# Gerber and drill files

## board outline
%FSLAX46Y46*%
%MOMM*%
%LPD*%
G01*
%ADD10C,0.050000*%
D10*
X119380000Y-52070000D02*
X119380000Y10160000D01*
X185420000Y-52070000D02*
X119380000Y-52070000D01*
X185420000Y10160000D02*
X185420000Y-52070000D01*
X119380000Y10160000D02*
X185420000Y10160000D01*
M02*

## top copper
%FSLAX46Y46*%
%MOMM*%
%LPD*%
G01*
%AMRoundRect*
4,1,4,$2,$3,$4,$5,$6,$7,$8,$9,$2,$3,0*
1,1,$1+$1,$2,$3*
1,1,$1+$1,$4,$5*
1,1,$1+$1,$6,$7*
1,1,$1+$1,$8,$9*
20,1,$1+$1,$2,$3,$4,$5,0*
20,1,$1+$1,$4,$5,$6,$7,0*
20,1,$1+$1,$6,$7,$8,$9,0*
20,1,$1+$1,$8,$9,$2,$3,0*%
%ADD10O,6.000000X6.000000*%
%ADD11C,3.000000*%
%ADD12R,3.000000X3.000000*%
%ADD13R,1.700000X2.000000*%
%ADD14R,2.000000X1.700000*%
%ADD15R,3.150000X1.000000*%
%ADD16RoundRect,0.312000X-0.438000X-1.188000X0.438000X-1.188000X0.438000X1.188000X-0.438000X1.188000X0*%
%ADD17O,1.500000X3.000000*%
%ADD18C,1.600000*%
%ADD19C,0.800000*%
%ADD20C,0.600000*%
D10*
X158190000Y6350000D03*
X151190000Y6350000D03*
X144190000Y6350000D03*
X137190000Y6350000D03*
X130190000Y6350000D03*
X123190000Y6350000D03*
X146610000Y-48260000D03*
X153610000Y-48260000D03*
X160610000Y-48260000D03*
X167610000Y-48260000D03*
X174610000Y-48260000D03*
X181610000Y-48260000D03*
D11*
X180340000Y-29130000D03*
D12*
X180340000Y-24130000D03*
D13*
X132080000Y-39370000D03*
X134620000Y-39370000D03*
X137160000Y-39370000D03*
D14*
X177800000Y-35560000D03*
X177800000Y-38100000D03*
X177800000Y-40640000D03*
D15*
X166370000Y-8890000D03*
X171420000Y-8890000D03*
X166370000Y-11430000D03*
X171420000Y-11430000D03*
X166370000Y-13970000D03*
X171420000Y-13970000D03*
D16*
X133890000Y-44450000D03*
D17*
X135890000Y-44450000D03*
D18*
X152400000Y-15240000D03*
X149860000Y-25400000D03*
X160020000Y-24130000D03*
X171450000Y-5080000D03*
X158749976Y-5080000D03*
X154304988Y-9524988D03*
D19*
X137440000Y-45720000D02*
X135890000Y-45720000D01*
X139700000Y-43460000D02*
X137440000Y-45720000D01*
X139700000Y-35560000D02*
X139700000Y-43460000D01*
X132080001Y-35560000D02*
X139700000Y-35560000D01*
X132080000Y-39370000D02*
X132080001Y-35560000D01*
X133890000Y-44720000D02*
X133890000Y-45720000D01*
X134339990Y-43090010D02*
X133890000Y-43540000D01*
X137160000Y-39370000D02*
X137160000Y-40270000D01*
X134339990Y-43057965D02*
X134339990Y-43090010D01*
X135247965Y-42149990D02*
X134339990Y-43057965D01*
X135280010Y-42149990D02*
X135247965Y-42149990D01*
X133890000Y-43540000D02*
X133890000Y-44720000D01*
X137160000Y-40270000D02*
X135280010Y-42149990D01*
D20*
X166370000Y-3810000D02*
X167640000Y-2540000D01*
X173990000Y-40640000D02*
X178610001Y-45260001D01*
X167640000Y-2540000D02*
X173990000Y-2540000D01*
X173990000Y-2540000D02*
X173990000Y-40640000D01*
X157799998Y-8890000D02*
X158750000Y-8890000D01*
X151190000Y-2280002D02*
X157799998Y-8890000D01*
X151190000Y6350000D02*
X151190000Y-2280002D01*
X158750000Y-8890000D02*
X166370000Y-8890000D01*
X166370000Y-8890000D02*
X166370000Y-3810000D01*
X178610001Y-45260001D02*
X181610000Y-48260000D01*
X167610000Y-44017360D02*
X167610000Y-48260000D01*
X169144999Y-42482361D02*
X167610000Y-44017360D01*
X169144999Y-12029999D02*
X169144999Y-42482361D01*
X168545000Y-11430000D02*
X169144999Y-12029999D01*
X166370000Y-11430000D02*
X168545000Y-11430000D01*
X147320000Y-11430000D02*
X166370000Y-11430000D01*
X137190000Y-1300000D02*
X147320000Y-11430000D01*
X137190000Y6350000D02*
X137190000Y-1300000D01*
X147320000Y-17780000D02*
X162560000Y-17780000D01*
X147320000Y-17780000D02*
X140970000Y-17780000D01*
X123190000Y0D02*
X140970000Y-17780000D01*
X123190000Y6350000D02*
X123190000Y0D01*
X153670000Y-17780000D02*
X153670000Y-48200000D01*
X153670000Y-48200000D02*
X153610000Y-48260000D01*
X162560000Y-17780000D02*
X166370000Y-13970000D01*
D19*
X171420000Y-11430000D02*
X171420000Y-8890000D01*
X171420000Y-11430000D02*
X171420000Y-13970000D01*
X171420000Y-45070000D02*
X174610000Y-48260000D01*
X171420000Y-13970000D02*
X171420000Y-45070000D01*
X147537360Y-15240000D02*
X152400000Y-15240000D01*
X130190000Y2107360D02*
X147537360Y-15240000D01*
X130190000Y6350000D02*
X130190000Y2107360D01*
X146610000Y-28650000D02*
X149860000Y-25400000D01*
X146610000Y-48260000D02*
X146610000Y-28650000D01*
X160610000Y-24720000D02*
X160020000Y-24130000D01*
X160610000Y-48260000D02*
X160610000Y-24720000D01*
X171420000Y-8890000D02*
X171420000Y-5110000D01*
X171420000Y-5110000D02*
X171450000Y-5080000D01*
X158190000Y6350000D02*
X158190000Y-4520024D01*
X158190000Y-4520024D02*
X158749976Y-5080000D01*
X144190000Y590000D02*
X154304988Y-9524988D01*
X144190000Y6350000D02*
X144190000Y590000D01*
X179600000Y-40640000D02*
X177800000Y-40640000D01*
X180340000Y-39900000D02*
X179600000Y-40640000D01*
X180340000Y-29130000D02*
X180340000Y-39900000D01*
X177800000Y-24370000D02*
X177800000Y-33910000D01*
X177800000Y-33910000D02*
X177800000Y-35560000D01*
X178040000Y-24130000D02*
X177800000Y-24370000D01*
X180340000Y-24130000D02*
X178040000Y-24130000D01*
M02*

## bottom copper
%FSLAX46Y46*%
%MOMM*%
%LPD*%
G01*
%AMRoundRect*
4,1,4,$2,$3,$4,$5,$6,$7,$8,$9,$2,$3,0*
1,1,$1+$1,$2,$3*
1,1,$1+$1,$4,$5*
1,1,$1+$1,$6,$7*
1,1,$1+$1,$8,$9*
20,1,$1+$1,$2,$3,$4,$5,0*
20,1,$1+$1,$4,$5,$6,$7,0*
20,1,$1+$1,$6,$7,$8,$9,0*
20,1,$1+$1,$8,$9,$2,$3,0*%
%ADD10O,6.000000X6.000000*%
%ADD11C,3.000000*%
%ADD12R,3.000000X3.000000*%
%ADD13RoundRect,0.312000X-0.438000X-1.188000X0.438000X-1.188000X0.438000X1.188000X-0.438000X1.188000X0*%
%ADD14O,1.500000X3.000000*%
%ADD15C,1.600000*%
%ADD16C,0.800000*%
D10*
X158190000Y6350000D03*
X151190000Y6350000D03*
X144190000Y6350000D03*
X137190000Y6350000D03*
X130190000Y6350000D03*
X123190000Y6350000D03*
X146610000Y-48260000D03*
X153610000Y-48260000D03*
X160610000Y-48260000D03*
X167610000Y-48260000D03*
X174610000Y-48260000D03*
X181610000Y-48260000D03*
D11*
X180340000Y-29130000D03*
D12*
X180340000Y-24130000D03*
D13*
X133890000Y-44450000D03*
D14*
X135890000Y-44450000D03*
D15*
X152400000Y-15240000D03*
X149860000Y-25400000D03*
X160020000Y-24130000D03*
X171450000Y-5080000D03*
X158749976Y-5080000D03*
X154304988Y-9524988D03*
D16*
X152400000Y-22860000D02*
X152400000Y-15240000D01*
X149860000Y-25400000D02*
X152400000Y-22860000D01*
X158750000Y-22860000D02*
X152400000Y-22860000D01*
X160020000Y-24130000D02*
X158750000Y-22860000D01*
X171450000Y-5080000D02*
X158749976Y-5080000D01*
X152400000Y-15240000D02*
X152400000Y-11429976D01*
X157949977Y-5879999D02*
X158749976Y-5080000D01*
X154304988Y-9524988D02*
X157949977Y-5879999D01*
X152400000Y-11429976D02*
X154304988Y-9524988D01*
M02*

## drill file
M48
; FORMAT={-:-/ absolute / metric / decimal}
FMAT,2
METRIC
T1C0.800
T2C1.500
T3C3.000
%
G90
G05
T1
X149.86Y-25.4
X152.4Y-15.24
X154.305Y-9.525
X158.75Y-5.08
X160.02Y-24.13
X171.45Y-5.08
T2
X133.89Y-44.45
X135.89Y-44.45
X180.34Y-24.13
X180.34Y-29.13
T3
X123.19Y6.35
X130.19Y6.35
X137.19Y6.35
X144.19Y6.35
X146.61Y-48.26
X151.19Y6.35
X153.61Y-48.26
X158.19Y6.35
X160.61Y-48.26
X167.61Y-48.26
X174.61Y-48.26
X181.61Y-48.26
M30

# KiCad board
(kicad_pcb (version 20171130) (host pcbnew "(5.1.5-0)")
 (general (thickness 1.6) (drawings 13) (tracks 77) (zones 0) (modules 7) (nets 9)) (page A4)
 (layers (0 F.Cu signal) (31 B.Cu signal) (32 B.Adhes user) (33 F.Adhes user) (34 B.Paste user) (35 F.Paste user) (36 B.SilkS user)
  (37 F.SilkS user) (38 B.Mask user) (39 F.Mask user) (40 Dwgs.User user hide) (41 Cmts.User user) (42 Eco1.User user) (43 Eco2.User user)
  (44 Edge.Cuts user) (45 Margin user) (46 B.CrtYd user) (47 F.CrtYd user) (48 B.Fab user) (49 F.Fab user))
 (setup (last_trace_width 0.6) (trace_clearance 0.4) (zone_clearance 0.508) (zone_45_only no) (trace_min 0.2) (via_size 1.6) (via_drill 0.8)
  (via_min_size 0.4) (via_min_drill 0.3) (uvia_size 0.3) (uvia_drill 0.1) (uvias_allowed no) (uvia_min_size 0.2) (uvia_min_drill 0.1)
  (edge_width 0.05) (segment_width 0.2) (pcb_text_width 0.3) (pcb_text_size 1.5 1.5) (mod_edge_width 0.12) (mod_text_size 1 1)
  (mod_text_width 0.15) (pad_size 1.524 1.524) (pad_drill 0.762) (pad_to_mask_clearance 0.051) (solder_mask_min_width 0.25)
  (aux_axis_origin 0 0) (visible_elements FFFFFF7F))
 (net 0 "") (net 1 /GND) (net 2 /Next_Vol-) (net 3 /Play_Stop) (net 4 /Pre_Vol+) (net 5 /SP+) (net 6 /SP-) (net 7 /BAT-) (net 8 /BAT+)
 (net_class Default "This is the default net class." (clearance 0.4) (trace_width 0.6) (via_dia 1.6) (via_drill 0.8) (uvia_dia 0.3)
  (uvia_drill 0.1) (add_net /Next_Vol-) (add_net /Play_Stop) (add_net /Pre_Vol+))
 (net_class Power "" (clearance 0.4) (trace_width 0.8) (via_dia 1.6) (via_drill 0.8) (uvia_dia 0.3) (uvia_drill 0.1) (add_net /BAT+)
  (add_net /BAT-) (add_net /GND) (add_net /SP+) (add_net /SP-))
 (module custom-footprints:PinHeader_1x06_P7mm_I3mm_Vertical (layer F.Cu) (at 123.19 -6.35 90)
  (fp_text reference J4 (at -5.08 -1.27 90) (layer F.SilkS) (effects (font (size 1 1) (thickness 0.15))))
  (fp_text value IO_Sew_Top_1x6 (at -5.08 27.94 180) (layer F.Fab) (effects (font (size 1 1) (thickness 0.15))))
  (pad 6 thru_hole oval (at 0 35 90) (size 6 6) (drill 3) (layers *.Cu *.Mask) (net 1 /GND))
  (pad 5 thru_hole oval (at 0 28 90) (size 6 6) (drill 3) (layers *.Cu *.Mask) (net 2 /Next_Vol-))
  (pad 4 thru_hole oval (at 0 21 90) (size 6 6) (drill 3) (layers *.Cu *.Mask) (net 1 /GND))
  (pad 3 thru_hole oval (at 0 14 90) (size 6 6) (drill 3) (layers *.Cu *.Mask) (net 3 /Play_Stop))
  (pad 2 thru_hole oval (at 0 7 90) (size 6 6) (drill 3) (layers *.Cu *.Mask) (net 1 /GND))
  (pad 1 thru_hole oval (at 0 0 90) (size 6 6) (drill 3) (layers *.Cu *.Mask) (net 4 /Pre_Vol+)))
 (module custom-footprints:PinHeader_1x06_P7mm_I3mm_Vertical (layer F.Cu) (at 181.61 48.26 270)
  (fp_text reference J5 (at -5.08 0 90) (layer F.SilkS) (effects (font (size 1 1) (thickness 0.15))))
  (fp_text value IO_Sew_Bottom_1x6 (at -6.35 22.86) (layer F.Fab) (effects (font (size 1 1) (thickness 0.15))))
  (pad 6 thru_hole oval (at 0 35 270) (size 6 6) (drill 3) (layers *.Cu *.Mask) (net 1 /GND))
  (pad 5 thru_hole oval (at 0 28 270) (size 6 6) (drill 3) (layers *.Cu *.Mask) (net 4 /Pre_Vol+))
  (pad 4 thru_hole oval (at 0 21 270) (size 6 6) (drill 3) (layers *.Cu *.Mask) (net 1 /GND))
  (pad 3 thru_hole oval (at 0 14 270) (size 6 6) (drill 3) (layers *.Cu *.Mask) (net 3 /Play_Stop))
  (pad 2 thru_hole oval (at 0 7 270) (size 6 6) (drill 3) (layers *.Cu *.Mask) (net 1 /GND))
  (pad 1 thru_hole oval (at 0 0 270) (size 6 6) (drill 3) (layers *.Cu *.Mask) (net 2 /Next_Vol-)))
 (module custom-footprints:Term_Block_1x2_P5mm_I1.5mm (layer F.Cu) (at 180.34 24.13 270)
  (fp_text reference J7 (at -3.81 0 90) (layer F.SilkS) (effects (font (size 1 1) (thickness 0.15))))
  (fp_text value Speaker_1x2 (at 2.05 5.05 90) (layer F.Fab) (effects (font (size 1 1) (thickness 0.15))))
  (pad 2 thru_hole circle (at 5 0 270) (size 3 3) (drill 1.5) (layers *.Cu *.Mask) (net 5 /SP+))
  (pad 1 thru_hole rect (at 0 0 270) (size 3 3) (drill 1.5) (layers *.Cu *.Mask) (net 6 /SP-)))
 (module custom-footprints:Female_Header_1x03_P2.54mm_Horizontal (layer F.Cu) (at 132.08 39.37 90)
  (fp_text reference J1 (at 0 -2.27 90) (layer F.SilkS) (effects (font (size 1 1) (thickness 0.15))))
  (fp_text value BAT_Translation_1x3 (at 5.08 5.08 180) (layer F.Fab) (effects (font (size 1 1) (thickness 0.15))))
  (pad 1 smd rect (at 0 0 90) (size 2 1.7) (layers F.Cu F.Paste F.Mask) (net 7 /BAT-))
  (pad 2 smd rect (at 0 2.54 90) (size 2 1.7) (layers F.Cu F.Paste F.Mask))
  (pad 3 smd rect (at 0 5.08 90) (size 2 1.7) (layers F.Cu F.Paste F.Mask) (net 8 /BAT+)))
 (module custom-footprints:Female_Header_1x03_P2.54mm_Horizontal (layer F.Cu) (at 177.8 35.56)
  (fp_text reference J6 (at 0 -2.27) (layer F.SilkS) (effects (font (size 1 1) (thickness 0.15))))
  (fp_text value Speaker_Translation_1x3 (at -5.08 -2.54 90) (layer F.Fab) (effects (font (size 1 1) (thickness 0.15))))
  (pad 1 smd rect (at 0 0) (size 2 1.7) (layers F.Cu F.Paste F.Mask) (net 6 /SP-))
  (pad 2 smd rect (at 0 2.54) (size 2 1.7) (layers F.Cu F.Paste F.Mask))
  (pad 3 smd rect (at 0 5.08) (size 2 1.7) (layers F.Cu F.Paste F.Mask) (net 5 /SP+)))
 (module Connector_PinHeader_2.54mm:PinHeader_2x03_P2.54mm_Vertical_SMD (layer F.Cu) (at 168.895 11.43)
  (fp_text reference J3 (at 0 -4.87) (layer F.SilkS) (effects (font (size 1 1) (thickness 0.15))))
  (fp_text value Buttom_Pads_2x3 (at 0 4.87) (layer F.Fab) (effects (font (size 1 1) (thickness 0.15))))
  (pad 1 smd rect (at -2.525 -2.54) (size 3.15 1) (layers F.Cu F.Paste F.Mask) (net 2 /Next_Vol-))
  (pad 2 smd rect (at 2.525 -2.54) (size 3.15 1) (layers F.Cu F.Paste F.Mask) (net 1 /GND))
  (pad 3 smd rect (at -2.525 0) (size 3.15 1) (layers F.Cu F.Paste F.Mask) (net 3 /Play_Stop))
  (pad 4 smd rect (at 2.525 0) (size 3.15 1) (layers F.Cu F.Paste F.Mask) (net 1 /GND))
  (pad 5 smd rect (at -2.525 2.54) (size 3.15 1) (layers F.Cu F.Paste F.Mask) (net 4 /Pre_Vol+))
  (pad 6 smd rect (at 2.525 2.54) (size 3.15 1) (layers F.Cu F.Paste F.Mask) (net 1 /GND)))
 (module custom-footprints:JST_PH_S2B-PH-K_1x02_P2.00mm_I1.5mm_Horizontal (layer F.Cu) (at 133.89 44.45)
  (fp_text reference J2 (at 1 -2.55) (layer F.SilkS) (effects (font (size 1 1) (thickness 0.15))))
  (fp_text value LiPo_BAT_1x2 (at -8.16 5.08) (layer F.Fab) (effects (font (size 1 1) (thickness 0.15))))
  (pad 1 thru_hole roundrect (at 0 0) (size 1.5 3) (drill 1.5) (layers *.Cu *.Mask) (roundrect_rratio 0.208) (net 8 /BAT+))
  (pad 2 thru_hole oval (at 2 0) (size 1.5 3) (drill 1.5) (layers *.Cu *.Mask) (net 7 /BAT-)))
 (gr_line (start 119.38 52.07) (end 119.38 -10.16) (layer Edge.Cuts) (width 0.05))
 (gr_line (start 185.42 52.07) (end 119.38 52.07) (layer Edge.Cuts) (width 0.05))
 (gr_line (start 185.42 -10.16) (end 185.42 52.07) (layer Edge.Cuts) (width 0.05))
 (gr_line (start 119.38 -10.16) (end 185.42 -10.16) (layer Edge.Cuts) (width 0.05))
 (segment (start 137.44 45.72) (end 135.89 45.72) (width 0.8) (layer F.Cu) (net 7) (status 20))
 (segment (start 139.7 43.46) (end 137.44 45.72) (width 0.8) (layer F.Cu) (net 7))
 (segment (start 139.7 35.56) (end 139.7 43.46) (width 0.8) (layer F.Cu) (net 7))
 (segment (start 132.080001 35.56) (end 139.7 35.56) (width 0.8) (layer F.Cu) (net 7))
 (segment (start 132.08 39.37) (end 132.080001 35.56) (width 0.8) (layer F.Cu) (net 7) (status 10))
 (segment (start 133.89 44.72) (end 133.89 45.72) (width 0.8) (layer F.Cu) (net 8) (status 30))
 (segment (start 134.33999 43.09001) (end 133.89 43.54) (width 0.8) (layer F.Cu) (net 8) (status 30))
 (segment (start 137.16 39.37) (end 137.16 40.27) (width 0.8) (layer F.Cu) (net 8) (status 30))
 (segment (start 134.33999 43.057965) (end 134.33999 43.09001) (width 0.8) (layer F.Cu) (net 8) (status 30))
 (segment (start 135.247965 42.14999) (end 134.33999 43.057965) (width 0.8) (layer F.Cu) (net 8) (status 20))
 (segment (start 135.28001 42.14999) (end 135.247965 42.14999) (width 0.8) (layer F.Cu) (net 8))
 (segment (start 133.89 43.54) (end 133.89 44.72) (width 0.8) (layer F.Cu) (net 8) (status 30))
 (segment (start 137.16 40.27) (end 135.28001 42.14999) (width 0.8) (layer F.Cu) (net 8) (status 10))
 (segment (start 166.37 3.81) (end 167.64 2.54) (width 0.6) (layer F.Cu) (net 2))
 (segment (start 173.99 40.64) (end 178.610001 45.260001) (width 0.6) (layer F.Cu) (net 2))
 (segment (start 167.64 2.54) (end 173.99 2.54) (width 0.6) (layer F.Cu) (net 2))
 (segment (start 173.99 2.54) (end 173.99 40.64) (width 0.6) (layer F.Cu) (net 2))
 (segment (start 157.799998 8.89) (end 158.75 8.89) (width 0.6) (layer F.Cu) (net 2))
 (segment (start 151.19 2.280002) (end 157.799998 8.89) (width 0.6) (layer F.Cu) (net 2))
 (segment (start 151.19 -6.35) (end 151.19 2.280002) (width 0.6) (layer F.Cu) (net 2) (status 10))
 (segment (start 158.75 8.89) (end 166.37 8.89) (width 0.6) (layer F.Cu) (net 2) (status 20))
 (segment (start 166.37 8.89) (end 166.37 3.81) (width 0.6) (layer F.Cu) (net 2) (status 10))
 (segment (start 178.610001 45.260001) (end 181.61 48.26) (width 0.6) (layer F.Cu) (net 2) (status 20))
 (segment (start 167.61 44.01736) (end 167.61 48.26) (width 0.6) (layer F.Cu) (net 3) (status 20))
 (segment (start 169.144999 42.482361) (end 167.61 44.01736) (width 0.6) (layer F.Cu) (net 3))
 (segment (start 169.144999 12.029999) (end 169.144999 42.482361) (width 0.6) (layer F.Cu) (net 3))
 (segment (start 168.545 11.43) (end 169.144999 12.029999) (width 0.6) (layer F.Cu) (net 3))
 (segment (start 166.37 11.43) (end 168.545 11.43) (width 0.6) (layer F.Cu) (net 3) (status 10))
 (segment (start 147.32 11.43) (end 166.37 11.43) (width 0.6) (layer F.Cu) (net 3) (status 20))
 (segment (start 137.19 1.3) (end 147.32 11.43) (width 0.6) (layer F.Cu) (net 3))
 (segment (start 137.19 -6.35) (end 137.19 1.3) (width 0.6) (layer F.Cu) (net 3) (status 10))
 (segment (start 147.32 17.78) (end 162.56 17.78) (width 0.6) (layer F.Cu) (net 4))
 (segment (start 147.32 17.78) (end 140.97 17.78) (width 0.6) (layer F.Cu) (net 4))
 (segment (start 123.19 0) (end 140.97 17.78) (width 0.6) (layer F.Cu) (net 4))
 (segment (start 123.19 -6.35) (end 123.19 0) (width 0.6) (layer F.Cu) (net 4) (status 10))
 (segment (start 153.67 17.78) (end 153.67 48.2) (width 0.6) (layer F.Cu) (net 4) (status 20))
 (segment (start 153.67 48.2) (end 153.61 48.26) (width 0.6) (layer F.Cu) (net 4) (status 30))
 (segment (start 162.56 17.78) (end 166.37 13.97) (width 0.6) (layer F.Cu) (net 4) (status 20))
 (segment (start 171.42 11.43) (end 171.42 8.89) (width 0.8) (layer F.Cu) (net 1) (status 30))
 (segment (start 171.42 11.43) (end 171.42 13.97) (width 0.8) (layer F.Cu) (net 1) (status 30))
 (segment (start 171.42 45.07) (end 174.61 48.26) (width 0.8) (layer F.Cu) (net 1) (status 20))
 (segment (start 171.42 13.97) (end 171.42 45.07) (width 0.8) (layer F.Cu) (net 1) (status 10))
 (segment (start 147.53736 15.24) (end 152.4 15.24) (width 0.8) (layer F.Cu) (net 1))
 (via (at 152.4 15.24) (size 1.6) (drill 0.8) (layers F.Cu B.Cu) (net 1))
 (segment (start 130.19 -2.10736) (end 147.53736 15.24) (width 0.8) (layer F.Cu) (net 1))
 (segment (start 130.19 -6.35) (end 130.19 -2.10736) (width 0.8) (layer F.Cu) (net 1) (status 10))
 (via (at 149.86 25.4) (size 1.6) (drill 0.8) (layers F.Cu B.Cu) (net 1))
 (segment (start 146.61 28.65) (end 149.86 25.4) (width 0.8) (layer F.Cu) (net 1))
 (segment (start 146.61 48.26) (end 146.61 28.65) (width 0.8) (layer F.Cu) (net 1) (status 10))
 (segment (start 152.4 22.86) (end 152.4 15.24) (width 0.8) (layer B.Cu) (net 1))
 (segment (start 149.86 25.4) (end 152.4 22.86) (width 0.8) (layer B.Cu) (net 1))
 (segment (start 160.61 24.72) (end 160.02 24.13) (width 0.8) (layer F.Cu) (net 1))
 (via (at 160.02 24.13) (size 1.6) (drill 0.8) (layers F.Cu B.Cu) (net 1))
 (segment (start 160.61 48.26) (end 160.61 24.72) (width 0.8) (layer F.Cu) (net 1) (status 10))
 (segment (start 158.75 22.86) (end 152.4 22.86) (width 0.8) (layer B.Cu) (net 1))
 (segment (start 160.02 24.13) (end 158.75 22.86) (width 0.8) (layer B.Cu) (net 1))
 (via (at 171.45 5.08) (size 1.6) (drill 0.8) (layers F.Cu B.Cu) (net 1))
 (segment (start 171.42 8.89) (end 171.42 5.11) (width 0.8) (layer F.Cu) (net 1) (status 10))
 (segment (start 171.42 5.11) (end 171.45 5.08) (width 0.8) (layer F.Cu) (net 1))
 (segment (start 171.45 5.08) (end 158.749976 5.08) (width 0.8) (layer B.Cu) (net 1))
 (via (at 158.749976 5.08) (size 1.6) (drill 0.8) (layers F.Cu B.Cu) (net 1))
 (segment (start 158.19 -6.35) (end 158.19 4.520024) (width 0.8) (layer F.Cu) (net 1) (status 10))
 (segment (start 152.4 15.24) (end 152.4 11.429976) (width 0.8) (layer B.Cu) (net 1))
 (segment (start 157.949977 5.879999) (end 158.749976 5.08) (width 0.8) (layer B.Cu) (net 1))
 (segment (start 158.19 4.520024) (end 158.749976 5.08) (width 0.8) (layer F.Cu) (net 1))
 (segment (start 144.19 -0.59) (end 154.304988 9.524988) (width 0.8) (layer F.Cu) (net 1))
 (segment (start 154.304988 9.524988) (end 157.949977 5.879999) (width 0.8) (layer B.Cu) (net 1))
 (via (at 154.304988 9.524988) (size 1.6) (drill 0.8) (layers F.Cu B.Cu) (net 1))
 (segment (start 144.19 -6.35) (end 144.19 -0.59) (width 0.8) (layer F.Cu) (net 1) (status 10))
 (segment (start 152.4 11.429976) (end 154.304988 9.524988) (width 0.8) (layer B.Cu) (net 1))
 (segment (start 179.6 40.64) (end 177.8 40.64) (width 0.8) (layer F.Cu) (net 5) (status 20))
 (segment (start 180.34 39.9) (end 179.6 40.64) (width 0.8) (layer F.Cu) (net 5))
 (segment (start 180.34 29.13) (end 180.34 39.9) (width 0.8) (layer F.Cu) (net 5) (status 10))
 (segment (start 177.8 24.37) (end 177.8 33.91) (width 0.8) (layer F.Cu) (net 6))
 (segment (start 177.8 33.91) (end 177.8 35.56) (width 0.8) (layer F.Cu) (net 6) (status 20))
 (segment (start 178.04 24.13) (end 177.8 24.37) (width 0.8) (layer F.Cu) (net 6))
 (segment (start 180.34 24.13) (end 178.04 24.13) (width 0.8) (layer F.Cu) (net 6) (status 10)))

